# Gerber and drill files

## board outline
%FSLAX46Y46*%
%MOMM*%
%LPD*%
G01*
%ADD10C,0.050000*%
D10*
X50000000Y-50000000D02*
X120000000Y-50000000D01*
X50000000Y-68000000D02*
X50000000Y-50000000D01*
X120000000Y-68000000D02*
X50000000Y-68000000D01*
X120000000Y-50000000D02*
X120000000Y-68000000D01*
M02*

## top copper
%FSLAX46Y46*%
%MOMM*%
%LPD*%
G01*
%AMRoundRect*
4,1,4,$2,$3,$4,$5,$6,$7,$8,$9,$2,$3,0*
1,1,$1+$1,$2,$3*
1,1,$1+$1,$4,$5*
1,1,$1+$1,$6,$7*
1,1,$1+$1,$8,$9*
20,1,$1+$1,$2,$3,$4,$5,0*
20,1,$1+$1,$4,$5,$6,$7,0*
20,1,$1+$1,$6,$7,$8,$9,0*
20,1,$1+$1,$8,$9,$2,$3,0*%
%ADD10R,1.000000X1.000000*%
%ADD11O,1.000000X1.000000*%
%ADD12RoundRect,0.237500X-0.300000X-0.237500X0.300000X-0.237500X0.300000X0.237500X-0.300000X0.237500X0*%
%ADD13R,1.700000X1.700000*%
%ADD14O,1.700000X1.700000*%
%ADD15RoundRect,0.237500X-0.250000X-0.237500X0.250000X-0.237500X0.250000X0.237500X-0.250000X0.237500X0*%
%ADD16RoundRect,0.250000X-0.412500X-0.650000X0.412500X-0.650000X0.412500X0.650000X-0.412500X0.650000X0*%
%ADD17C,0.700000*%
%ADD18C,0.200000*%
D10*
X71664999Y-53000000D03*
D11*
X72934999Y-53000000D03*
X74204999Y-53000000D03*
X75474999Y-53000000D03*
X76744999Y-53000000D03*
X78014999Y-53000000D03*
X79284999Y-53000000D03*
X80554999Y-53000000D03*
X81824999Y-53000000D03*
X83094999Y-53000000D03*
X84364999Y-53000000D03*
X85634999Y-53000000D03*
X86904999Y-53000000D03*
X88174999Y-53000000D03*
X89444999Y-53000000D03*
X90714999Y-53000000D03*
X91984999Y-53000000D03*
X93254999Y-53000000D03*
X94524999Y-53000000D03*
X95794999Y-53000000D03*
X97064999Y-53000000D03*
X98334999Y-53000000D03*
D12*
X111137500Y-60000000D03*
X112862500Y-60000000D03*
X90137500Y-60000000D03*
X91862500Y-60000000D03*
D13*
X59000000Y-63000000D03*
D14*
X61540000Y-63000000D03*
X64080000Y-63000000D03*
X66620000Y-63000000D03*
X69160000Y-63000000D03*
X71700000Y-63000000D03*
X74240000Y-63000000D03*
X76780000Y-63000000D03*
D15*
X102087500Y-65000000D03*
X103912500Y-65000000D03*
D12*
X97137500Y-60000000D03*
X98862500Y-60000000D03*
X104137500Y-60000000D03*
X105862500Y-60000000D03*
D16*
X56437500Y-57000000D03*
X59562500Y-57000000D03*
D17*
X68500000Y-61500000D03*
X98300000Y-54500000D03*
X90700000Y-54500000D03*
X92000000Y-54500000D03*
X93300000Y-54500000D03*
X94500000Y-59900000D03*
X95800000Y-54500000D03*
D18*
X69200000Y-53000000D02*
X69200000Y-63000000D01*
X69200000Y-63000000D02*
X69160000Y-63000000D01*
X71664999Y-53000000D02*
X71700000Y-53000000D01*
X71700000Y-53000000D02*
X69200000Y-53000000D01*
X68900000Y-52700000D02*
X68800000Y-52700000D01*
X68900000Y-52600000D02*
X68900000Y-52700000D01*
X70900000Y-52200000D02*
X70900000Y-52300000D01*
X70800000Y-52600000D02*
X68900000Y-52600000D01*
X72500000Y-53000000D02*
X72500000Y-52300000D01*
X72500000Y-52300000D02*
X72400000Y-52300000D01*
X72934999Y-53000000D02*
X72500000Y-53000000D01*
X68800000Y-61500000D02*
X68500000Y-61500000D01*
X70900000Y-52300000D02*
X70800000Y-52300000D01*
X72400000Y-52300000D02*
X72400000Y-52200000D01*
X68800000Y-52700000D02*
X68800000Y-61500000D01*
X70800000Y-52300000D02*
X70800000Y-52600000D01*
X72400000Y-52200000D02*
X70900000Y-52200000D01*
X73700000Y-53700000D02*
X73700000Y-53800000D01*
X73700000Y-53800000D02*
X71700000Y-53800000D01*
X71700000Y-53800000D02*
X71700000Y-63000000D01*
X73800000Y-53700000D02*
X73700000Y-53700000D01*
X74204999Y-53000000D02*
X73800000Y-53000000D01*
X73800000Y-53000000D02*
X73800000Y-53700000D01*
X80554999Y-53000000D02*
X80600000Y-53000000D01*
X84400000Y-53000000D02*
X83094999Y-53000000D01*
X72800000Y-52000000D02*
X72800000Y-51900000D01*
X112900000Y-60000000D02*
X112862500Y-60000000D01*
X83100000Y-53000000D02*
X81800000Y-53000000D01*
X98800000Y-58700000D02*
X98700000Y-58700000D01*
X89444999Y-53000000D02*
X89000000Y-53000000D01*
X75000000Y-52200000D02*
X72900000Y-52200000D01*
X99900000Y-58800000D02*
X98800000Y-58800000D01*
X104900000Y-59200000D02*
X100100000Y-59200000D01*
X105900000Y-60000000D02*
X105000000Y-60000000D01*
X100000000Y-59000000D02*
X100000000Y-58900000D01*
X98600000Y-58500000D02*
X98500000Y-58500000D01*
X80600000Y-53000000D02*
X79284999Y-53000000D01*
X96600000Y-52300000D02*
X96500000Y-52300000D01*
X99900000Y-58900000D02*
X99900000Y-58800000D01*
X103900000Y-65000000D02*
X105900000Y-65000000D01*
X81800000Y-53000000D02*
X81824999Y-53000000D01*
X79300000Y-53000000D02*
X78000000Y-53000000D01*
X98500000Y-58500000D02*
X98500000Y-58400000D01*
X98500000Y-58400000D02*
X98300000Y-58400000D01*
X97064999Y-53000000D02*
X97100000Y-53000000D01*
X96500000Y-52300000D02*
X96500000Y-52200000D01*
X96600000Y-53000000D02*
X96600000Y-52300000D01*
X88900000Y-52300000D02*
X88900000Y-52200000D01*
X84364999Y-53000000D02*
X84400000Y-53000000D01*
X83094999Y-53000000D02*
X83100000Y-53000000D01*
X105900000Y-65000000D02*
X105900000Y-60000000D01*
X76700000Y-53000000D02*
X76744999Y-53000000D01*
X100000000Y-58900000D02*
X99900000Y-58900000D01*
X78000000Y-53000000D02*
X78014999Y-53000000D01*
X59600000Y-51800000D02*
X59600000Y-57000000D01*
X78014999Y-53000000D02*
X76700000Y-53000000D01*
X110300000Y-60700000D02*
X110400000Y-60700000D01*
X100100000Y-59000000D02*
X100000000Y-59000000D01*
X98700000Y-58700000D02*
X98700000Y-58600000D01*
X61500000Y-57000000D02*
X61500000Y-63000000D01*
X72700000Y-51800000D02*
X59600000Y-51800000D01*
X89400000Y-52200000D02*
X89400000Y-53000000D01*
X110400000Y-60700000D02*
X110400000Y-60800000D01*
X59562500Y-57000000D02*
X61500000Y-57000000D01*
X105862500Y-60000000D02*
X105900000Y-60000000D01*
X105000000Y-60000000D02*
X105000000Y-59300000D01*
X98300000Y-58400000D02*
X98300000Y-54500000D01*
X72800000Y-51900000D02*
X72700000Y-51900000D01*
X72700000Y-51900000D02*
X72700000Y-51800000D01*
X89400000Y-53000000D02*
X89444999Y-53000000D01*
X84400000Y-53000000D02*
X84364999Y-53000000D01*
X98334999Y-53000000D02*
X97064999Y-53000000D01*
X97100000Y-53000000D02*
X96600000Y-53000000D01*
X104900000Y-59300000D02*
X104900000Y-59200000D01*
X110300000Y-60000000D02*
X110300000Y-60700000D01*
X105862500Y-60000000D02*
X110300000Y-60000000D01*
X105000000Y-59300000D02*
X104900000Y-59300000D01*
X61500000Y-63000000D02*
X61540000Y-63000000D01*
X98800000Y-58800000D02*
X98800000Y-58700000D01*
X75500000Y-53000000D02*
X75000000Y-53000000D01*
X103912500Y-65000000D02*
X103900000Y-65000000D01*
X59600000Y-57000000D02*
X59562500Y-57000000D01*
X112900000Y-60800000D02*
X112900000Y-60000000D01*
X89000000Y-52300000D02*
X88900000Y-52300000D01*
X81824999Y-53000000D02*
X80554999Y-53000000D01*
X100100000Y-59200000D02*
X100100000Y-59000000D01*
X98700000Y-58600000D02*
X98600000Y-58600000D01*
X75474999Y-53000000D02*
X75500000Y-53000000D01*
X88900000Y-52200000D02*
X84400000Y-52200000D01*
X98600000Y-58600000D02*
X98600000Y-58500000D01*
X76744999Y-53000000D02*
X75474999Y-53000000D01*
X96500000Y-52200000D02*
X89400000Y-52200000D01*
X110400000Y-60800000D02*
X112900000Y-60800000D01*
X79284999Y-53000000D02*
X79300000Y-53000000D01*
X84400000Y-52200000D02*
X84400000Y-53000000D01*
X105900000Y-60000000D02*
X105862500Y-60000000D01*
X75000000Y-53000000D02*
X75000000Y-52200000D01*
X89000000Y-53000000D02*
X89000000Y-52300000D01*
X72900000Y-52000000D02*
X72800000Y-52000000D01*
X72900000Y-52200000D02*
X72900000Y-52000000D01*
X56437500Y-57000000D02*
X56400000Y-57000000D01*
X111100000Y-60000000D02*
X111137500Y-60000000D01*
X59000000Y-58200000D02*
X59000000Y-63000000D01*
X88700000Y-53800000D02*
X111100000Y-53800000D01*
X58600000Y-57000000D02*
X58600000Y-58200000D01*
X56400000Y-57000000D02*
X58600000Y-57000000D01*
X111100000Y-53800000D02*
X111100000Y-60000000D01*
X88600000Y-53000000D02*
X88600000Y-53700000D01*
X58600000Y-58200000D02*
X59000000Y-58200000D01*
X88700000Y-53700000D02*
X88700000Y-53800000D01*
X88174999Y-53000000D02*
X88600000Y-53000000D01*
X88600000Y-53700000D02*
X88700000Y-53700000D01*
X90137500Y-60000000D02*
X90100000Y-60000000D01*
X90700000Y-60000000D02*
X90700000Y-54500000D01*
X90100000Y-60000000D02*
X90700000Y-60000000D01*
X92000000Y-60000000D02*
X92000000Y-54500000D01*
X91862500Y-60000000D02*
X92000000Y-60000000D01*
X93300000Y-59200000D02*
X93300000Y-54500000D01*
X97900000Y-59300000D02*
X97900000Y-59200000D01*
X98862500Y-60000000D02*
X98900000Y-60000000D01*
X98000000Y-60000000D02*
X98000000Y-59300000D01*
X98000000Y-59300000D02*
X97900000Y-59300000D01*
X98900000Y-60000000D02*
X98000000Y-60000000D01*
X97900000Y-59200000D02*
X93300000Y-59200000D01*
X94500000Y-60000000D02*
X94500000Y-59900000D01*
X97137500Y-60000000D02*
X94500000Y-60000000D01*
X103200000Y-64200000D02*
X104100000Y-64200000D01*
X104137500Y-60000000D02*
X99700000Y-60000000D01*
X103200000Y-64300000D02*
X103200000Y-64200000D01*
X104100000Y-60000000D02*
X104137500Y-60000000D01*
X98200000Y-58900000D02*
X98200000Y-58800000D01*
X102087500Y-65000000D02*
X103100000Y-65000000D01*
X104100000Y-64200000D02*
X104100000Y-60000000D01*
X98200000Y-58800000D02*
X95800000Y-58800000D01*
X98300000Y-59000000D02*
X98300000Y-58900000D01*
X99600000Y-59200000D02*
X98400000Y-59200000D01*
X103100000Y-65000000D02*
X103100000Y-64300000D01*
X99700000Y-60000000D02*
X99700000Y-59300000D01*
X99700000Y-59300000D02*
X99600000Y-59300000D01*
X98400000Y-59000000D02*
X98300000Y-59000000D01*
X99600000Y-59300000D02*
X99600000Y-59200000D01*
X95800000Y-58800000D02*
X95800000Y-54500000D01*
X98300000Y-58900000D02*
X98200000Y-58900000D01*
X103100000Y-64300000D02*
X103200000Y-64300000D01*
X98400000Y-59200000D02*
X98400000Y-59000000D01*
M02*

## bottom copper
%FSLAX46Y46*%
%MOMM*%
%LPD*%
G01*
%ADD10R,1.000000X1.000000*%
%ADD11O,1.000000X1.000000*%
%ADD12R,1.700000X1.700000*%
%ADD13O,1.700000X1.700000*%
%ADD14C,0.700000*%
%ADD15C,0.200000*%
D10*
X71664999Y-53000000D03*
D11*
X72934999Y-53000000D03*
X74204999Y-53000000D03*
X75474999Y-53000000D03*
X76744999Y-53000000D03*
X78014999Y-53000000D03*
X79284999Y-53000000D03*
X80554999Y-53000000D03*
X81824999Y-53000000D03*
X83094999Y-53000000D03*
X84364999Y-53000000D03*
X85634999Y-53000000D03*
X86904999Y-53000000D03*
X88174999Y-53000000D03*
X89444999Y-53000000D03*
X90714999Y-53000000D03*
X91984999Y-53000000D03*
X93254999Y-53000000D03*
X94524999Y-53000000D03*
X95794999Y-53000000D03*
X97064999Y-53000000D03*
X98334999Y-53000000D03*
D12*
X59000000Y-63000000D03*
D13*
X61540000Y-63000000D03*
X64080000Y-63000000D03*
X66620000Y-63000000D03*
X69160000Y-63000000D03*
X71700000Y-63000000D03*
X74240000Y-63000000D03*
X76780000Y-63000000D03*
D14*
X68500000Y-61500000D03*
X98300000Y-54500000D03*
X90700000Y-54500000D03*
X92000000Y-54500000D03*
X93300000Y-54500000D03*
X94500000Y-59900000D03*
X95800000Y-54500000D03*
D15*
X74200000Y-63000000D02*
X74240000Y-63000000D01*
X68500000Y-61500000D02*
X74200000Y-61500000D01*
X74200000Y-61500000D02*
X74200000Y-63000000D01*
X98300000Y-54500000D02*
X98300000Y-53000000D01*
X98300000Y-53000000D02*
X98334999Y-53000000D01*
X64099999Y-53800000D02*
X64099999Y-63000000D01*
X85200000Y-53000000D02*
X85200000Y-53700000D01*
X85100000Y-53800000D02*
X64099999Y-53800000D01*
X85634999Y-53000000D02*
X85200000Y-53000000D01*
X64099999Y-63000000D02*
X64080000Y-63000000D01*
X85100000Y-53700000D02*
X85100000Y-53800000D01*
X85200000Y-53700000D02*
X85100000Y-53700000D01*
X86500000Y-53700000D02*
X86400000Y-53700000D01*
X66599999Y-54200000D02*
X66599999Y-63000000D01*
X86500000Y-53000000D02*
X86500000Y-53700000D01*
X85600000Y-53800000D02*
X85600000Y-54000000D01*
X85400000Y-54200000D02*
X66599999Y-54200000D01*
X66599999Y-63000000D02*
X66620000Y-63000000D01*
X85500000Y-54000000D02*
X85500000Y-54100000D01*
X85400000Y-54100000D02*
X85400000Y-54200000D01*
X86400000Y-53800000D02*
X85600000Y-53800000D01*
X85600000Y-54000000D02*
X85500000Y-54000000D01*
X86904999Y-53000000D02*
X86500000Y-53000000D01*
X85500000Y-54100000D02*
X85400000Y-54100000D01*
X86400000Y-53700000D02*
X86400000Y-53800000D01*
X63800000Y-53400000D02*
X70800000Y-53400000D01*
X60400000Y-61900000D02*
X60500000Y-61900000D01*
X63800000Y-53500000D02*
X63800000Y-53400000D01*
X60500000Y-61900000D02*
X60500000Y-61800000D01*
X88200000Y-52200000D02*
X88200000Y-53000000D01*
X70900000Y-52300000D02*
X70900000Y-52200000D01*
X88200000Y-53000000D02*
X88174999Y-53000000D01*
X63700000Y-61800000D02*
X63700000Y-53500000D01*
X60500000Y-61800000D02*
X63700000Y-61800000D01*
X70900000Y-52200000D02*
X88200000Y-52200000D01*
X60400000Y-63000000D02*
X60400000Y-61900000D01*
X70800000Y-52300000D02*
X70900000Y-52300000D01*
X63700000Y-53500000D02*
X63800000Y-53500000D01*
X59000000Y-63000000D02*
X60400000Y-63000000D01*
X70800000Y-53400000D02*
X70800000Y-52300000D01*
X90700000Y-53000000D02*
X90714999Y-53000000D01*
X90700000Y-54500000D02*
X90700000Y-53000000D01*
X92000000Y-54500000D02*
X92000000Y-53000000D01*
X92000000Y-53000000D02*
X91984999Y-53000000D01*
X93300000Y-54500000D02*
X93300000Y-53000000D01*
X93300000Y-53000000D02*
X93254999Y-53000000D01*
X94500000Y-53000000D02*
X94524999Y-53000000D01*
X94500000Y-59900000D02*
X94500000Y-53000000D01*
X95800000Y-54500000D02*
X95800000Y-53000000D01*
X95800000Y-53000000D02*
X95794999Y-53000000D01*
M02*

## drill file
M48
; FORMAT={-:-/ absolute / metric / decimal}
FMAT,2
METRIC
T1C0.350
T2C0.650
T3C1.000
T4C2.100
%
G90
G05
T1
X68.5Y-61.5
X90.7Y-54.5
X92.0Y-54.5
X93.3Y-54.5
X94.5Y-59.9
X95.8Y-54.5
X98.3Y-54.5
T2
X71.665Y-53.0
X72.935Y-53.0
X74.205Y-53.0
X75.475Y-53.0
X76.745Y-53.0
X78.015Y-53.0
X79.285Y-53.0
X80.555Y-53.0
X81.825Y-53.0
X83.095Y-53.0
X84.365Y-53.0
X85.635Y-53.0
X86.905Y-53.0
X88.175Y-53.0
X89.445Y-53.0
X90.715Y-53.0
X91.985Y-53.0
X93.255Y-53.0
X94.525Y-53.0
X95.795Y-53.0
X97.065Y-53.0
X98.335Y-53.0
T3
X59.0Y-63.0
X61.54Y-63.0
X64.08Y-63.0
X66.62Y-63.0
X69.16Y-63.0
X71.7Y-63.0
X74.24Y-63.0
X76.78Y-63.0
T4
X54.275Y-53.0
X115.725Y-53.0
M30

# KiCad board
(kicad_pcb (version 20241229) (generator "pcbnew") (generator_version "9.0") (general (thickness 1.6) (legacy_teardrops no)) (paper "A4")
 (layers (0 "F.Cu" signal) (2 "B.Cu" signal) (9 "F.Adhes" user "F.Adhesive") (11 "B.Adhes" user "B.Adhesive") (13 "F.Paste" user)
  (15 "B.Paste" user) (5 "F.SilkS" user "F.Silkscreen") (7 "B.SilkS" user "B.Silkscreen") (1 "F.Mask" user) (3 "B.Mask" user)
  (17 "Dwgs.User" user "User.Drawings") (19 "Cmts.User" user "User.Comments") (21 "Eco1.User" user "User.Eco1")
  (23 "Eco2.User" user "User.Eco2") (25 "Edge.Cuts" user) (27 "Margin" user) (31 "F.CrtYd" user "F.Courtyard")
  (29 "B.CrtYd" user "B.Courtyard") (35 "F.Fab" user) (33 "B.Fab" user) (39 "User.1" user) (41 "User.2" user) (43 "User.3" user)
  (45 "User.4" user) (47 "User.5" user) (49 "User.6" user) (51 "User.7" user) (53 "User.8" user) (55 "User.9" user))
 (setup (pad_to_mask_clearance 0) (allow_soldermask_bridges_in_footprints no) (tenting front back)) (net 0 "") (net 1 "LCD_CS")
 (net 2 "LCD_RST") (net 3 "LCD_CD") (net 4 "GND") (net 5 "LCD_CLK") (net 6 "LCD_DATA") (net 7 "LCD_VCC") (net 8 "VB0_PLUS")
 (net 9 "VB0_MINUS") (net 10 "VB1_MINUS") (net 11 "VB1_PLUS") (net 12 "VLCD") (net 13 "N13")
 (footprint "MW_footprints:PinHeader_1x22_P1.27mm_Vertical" (layer "F.Cu") (at 71.664999 53 90)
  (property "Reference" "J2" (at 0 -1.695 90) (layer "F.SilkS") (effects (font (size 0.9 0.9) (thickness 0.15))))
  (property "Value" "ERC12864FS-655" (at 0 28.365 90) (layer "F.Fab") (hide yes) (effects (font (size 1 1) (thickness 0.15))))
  (pad "1" thru_hole rect (at 0 0 90) (size 1 1) (drill 0.65) (layers "*.Cu" "*.Mask") (remove_unused_layers no) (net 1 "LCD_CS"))
  (pad "2" thru_hole oval (at 0 1.27 90) (size 1 1) (drill 0.65) (layers "*.Cu" "*.Mask") (remove_unused_layers no) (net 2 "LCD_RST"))
  (pad "3" thru_hole oval (at 0 2.54 90) (size 1 1) (drill 0.65) (layers "*.Cu" "*.Mask") (remove_unused_layers no) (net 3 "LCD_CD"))
  (pad "4" thru_hole oval (at 0 3.81 90) (size 1 1) (drill 0.65) (layers "*.Cu" "*.Mask") (remove_unused_layers no) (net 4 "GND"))
  (pad "5" thru_hole oval (at 0 5.08 90) (size 1 1) (drill 0.65) (layers "*.Cu" "*.Mask") (remove_unused_layers no) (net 4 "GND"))
  (pad "6" thru_hole oval (at 0 6.35 90) (size 1 1) (drill 0.65) (layers "*.Cu" "*.Mask") (remove_unused_layers no) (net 4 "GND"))
  (pad "7" thru_hole oval (at 0 7.62 90) (size 1 1) (drill 0.65) (layers "*.Cu" "*.Mask") (remove_unused_layers no) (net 4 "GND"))
  (pad "8" thru_hole oval (at 0 8.89 90) (size 1 1) (drill 0.65) (layers "*.Cu" "*.Mask") (remove_unused_layers no) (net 4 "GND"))
  (pad "9" thru_hole oval (at 0 10.16 90) (size 1 1) (drill 0.65) (layers "*.Cu" "*.Mask") (remove_unused_layers no) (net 4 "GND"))
  (pad "10" thru_hole oval (at 0 11.43 90) (size 1 1) (drill 0.65) (layers "*.Cu" "*.Mask") (remove_unused_layers no) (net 4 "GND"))
  (pad "11" thru_hole oval (at 0 12.7 90) (size 1 1) (drill 0.65) (layers "*.Cu" "*.Mask") (remove_unused_layers no) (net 4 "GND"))
  (pad "12" thru_hole oval (at 0 13.97 90) (size 1 1) (drill 0.65) (layers "*.Cu" "*.Mask") (remove_unused_layers no) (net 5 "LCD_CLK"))
  (pad "13" thru_hole oval (at 0 15.24 90) (size 1 1) (drill 0.65) (layers "*.Cu" "*.Mask") (remove_unused_layers no) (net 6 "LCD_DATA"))
  (pad "14" thru_hole oval (at 0 16.51 90) (size 1 1) (drill 0.65) (layers "*.Cu" "*.Mask") (remove_unused_layers no) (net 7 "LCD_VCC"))
  (pad "15" thru_hole oval (at 0 17.78 90) (size 1 1) (drill 0.65) (layers "*.Cu" "*.Mask") (remove_unused_layers no) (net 4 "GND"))
  (pad "16" thru_hole oval (at 0 19.05 90) (size 1 1) (drill 0.65) (layers "*.Cu" "*.Mask") (remove_unused_layers no) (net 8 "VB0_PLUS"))
  (pad "17" thru_hole oval (at 0 20.32 90) (size 1 1) (drill 0.65) (layers "*.Cu" "*.Mask") (remove_unused_layers no) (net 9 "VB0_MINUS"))
  (pad "18" thru_hole oval (at 0 21.59 90) (size 1 1) (drill 0.65) (layers "*.Cu" "*.Mask") (remove_unused_layers no) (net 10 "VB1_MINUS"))
  (pad "19" thru_hole oval (at 0 22.86 90) (size 1 1) (drill 0.65) (layers "*.Cu" "*.Mask") (remove_unused_layers no) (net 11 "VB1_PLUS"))
  (pad "20" thru_hole oval (at 0 24.13 90) (size 1 1) (drill 0.65) (layers "*.Cu" "*.Mask") (remove_unused_layers no) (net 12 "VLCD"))
  (pad "21" thru_hole oval (at 0 25.4 90) (size 1 1) (drill 0.65) (layers "*.Cu" "*.Mask") (remove_unused_layers no) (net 4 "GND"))
  (pad "22" thru_hole oval (at 0 26.67 90) (size 1 1) (drill 0.65) (layers "*.Cu" "*.Mask") (remove_unused_layers no) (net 4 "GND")))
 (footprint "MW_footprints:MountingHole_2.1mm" (layer "F.Cu") (at 54.275 53)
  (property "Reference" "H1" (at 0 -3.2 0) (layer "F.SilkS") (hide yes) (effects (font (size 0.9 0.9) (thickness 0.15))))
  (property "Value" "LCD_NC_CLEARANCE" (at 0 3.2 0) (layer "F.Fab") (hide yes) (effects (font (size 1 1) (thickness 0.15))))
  (pad "" np_thru_hole circle (at 0 0) (size 2.1 2.1) (drill 2.1) (layers "*.Cu" "*.Mask")))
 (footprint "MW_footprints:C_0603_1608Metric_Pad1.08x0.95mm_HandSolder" (layer "F.Cu") (at 112 60)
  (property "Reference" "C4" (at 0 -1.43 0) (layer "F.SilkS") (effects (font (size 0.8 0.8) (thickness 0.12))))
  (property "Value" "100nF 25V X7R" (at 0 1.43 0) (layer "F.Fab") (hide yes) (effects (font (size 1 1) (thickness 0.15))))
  (pad "1" smd roundrect (at -0.8625 0) (size 1.075 0.95) (layers "F.Cu" "F.Mask" "F.Paste") (roundrect_rratio 0.25) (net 7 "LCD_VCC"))
  (pad "2" smd roundrect (at 0.8625 0) (size 1.075 0.95) (layers "F.Cu" "F.Mask" "F.Paste") (roundrect_rratio 0.25) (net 4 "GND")))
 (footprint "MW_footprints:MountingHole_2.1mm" (layer "F.Cu") (at 115.725 53)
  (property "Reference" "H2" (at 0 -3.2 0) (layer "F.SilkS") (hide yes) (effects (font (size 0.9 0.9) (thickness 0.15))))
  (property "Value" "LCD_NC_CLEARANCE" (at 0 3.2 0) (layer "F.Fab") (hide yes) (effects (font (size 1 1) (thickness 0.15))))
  (pad "" np_thru_hole circle (at 0 0) (size 2.1 2.1) (drill 2.1) (layers "*.Cu" "*.Mask")))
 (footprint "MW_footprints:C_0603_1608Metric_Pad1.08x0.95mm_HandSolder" (layer "F.Cu") (at 91 60)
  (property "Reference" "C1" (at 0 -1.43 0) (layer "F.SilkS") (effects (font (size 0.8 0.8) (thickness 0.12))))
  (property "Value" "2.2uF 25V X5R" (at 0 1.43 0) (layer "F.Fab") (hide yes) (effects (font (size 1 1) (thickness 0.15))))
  (pad "1" smd roundrect (at -0.8625 0) (size 1.075 0.95) (layers "F.Cu" "F.Mask" "F.Paste") (roundrect_rratio 0.25) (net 8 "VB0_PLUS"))
  (pad "2" smd roundrect (at 0.8625 0) (size 1.075 0.95) (layers "F.Cu" "F.Mask" "F.Paste") (roundrect_rratio 0.25) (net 9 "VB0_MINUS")))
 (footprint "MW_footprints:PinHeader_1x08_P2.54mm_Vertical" (layer "F.Cu") (at 59 63 90)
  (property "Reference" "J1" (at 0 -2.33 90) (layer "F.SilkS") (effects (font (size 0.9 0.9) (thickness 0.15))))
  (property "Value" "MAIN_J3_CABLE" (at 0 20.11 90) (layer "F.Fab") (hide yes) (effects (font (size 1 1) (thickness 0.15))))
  (pad "1" thru_hole rect (at 0 0 90) (size 1.7 1.7) (drill 1) (layers "*.Cu" "*.Mask") (remove_unused_layers no) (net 7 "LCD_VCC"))
  (pad "2" thru_hole oval (at 0 2.54 90) (size 1.7 1.7) (drill 1) (layers "*.Cu" "*.Mask") (remove_unused_layers no) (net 4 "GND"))
  (pad "3" thru_hole oval (at 0 5.08 90) (size 1.7 1.7) (drill 1) (layers "*.Cu" "*.Mask") (remove_unused_layers no) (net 5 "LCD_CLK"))
  (pad "4" thru_hole oval (at 0 7.62 90) (size 1.7 1.7) (drill 1) (layers "*.Cu" "*.Mask") (remove_unused_layers no) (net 6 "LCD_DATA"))
  (pad "5" thru_hole oval (at 0 10.16 90) (size 1.7 1.7) (drill 1) (layers "*.Cu" "*.Mask") (remove_unused_layers no) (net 1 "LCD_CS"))
  (pad "6" thru_hole oval (at 0 12.7 90) (size 1.7 1.7) (drill 1) (layers "*.Cu" "*.Mask") (remove_unused_layers no) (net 3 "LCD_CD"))
  (pad "7" thru_hole oval (at 0 15.24 90) (size 1.7 1.7) (drill 1) (layers "*.Cu" "*.Mask") (remove_unused_layers no) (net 2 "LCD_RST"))
  (pad "8" thru_hole oval (at 0 17.78 90) (size 1.7 1.7) (drill 1) (layers "*.Cu" "*.Mask") (remove_unused_layers no) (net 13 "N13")))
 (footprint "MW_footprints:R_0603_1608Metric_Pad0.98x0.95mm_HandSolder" (layer "F.Cu") (at 103 65)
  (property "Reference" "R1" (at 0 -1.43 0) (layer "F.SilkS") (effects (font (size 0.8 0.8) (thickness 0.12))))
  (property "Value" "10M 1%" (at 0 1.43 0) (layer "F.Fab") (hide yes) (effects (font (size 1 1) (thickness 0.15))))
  (pad "1" smd roundrect (at -0.9125 0) (size 0.975 0.95) (layers "F.Cu" "F.Mask" "F.Paste") (roundrect_rratio 0.25) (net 12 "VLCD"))
  (pad "2" smd roundrect (at 0.9125 0) (size 0.975 0.95) (layers "F.Cu" "F.Mask" "F.Paste") (roundrect_rratio 0.25) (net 4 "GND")))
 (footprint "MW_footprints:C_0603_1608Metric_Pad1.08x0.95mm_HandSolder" (layer "F.Cu") (at 98 60)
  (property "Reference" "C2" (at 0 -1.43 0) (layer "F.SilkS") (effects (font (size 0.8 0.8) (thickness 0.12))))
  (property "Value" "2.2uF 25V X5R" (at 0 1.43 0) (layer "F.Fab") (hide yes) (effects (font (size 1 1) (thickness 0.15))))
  (pad "1" smd roundrect (at -0.8625 0) (size 1.075 0.95) (layers "F.Cu" "F.Mask" "F.Paste") (roundrect_rratio 0.25) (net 11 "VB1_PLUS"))
  (pad "2" smd roundrect (at 0.8625 0) (size 1.075 0.95) (layers "F.Cu" "F.Mask" "F.Paste") (roundrect_rratio 0.25) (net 10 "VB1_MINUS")))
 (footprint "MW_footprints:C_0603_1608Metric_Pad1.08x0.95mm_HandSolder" (layer "F.Cu") (at 105 60)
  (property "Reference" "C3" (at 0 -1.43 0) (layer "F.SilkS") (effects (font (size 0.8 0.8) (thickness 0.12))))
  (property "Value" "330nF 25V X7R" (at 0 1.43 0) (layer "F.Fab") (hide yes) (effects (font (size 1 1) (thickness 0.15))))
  (pad "1" smd roundrect (at -0.8625 0) (size 1.075 0.95) (layers "F.Cu" "F.Mask" "F.Paste") (roundrect_rratio 0.25) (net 12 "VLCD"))
  (pad "2" smd roundrect (at 0.8625 0) (size 1.075 0.95) (layers "F.Cu" "F.Mask" "F.Paste") (roundrect_rratio 0.25) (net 4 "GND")))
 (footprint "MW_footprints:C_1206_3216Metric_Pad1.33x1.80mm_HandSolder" (layer "F.Cu") (at 58 57)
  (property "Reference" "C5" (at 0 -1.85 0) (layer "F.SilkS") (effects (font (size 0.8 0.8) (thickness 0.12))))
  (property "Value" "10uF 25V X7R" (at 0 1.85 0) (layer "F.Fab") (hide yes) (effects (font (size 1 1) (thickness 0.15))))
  (pad "1" smd roundrect (at -1.5625 0) (size 1.325 1.8) (layers "F.Cu" "F.Mask" "F.Paste") (roundrect_rratio 0.188679) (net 7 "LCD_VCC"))
  (pad "2" smd roundrect (at 1.5625 0) (size 1.325 1.8) (layers "F.Cu" "F.Mask" "F.Paste") (roundrect_rratio 0.188679) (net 4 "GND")))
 (gr_line (start 50 50) (end 120 50) (stroke (width 0.05) (type default)) (layer "Edge.Cuts"))
 (gr_line (start 50 68) (end 50 50) (stroke (width 0.05) (type default)) (layer "Edge.Cuts"))
 (gr_line (start 120 68) (end 50 68) (stroke (width 0.05) (type default)) (layer "Edge.Cuts"))
 (gr_line (start 120 50) (end 120 68) (stroke (width 0.05) (type default)) (layer "Edge.Cuts"))
 (segment (start 69.2 53) (end 69.2 63) (width 0.2) (layer "F.Cu") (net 1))
 (segment (start 69.2 63) (end 69.16 63) (width 0.2) (layer "F.Cu") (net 1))
 (segment (start 71.664999 53) (end 71.7 53) (width 0.2) (layer "F.Cu") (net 1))
 (segment (start 71.7 53) (end 69.2 53) (width 0.2) (layer "F.Cu") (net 1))
 (segment (start 68.9 52.7) (end 68.8 52.7) (width 0.2) (layer "F.Cu") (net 2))
 (segment (start 68.9 52.6) (end 68.9 52.7) (width 0.2) (layer "F.Cu") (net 2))
 (segment (start 70.9 52.2) (end 70.9 52.3) (width 0.2) (layer "F.Cu") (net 2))
 (segment (start 70.8 52.6) (end 68.9 52.6) (width 0.2) (layer "F.Cu") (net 2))
 (segment (start 72.5 53) (end 72.5 52.3) (width 0.2) (layer "F.Cu") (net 2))
 (segment (start 72.5 52.3) (end 72.4 52.3) (width 0.2) (layer "F.Cu") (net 2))
 (segment (start 72.934999 53) (end 72.5 53) (width 0.2) (layer "F.Cu") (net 2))
 (segment (start 68.8 61.5) (end 68.5 61.5) (width 0.2) (layer "F.Cu") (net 2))
 (segment (start 70.9 52.3) (end 70.8 52.3) (width 0.2) (layer "F.Cu") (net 2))
 (segment (start 72.4 52.3) (end 72.4 52.2) (width 0.2) (layer "F.Cu") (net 2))
 (segment (start 68.8 52.7) (end 68.8 61.5) (width 0.2) (layer "F.Cu") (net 2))
 (segment (start 70.8 52.3) (end 70.8 52.6) (width 0.2) (layer "F.Cu") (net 2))
 (segment (start 72.4 52.2) (end 70.9 52.2) (width 0.2) (layer "F.Cu") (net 2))
 (via (at 68.5 61.5) (size 0.7) (drill 0.35) (layers "F.Cu" "B.Cu") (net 2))
 (segment (start 74.2 63) (end 74.24 63) (width 0.2) (layer "B.Cu") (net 2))
 (segment (start 68.5 61.5) (end 74.2 61.5) (width 0.2) (layer "B.Cu") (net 2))
 (segment (start 74.2 61.5) (end 74.2 63) (width 0.2) (layer "B.Cu") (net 2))
 (segment (start 73.7 53.7) (end 73.7 53.8) (width 0.2) (layer "F.Cu") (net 3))
 (segment (start 73.7 53.8) (end 71.7 53.8) (width 0.2) (layer "F.Cu") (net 3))
 (segment (start 71.7 53.8) (end 71.7 63) (width 0.2) (layer "F.Cu") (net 3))
 (segment (start 73.8 53.7) (end 73.7 53.7) (width 0.2) (layer "F.Cu") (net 3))
 (segment (start 74.204999 53) (end 73.8 53) (width 0.2) (layer "F.Cu") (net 3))
 (segment (start 73.8 53) (end 73.8 53.7) (width 0.2) (layer "F.Cu") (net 3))
 (segment (start 80.554999 53) (end 80.6 53) (width 0.2) (layer "F.Cu") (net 4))
 (segment (start 84.4 53) (end 83.094999 53) (width 0.2) (layer "F.Cu") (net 4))
 (segment (start 72.8 52) (end 72.8 51.9) (width 0.2) (layer "F.Cu") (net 4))
 (segment (start 112.9 60) (end 112.8625 60) (width 0.2) (layer "F.Cu") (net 4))
 (segment (start 83.1 53) (end 81.8 53) (width 0.2) (layer "F.Cu") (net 4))
 (segment (start 98.8 58.7) (end 98.7 58.7) (width 0.2) (layer "F.Cu") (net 4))
 (segment (start 89.444999 53) (end 89 53) (width 0.2) (layer "F.Cu") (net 4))
 (segment (start 75 52.2) (end 72.9 52.2) (width 0.2) (layer "F.Cu") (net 4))
 (segment (start 99.9 58.8) (end 98.8 58.8) (width 0.2) (layer "F.Cu") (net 4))
 (segment (start 104.9 59.2) (end 100.1 59.2) (width 0.2) (layer "F.Cu") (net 4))
 (segment (start 105.9 60) (end 105 60) (width 0.2) (layer "F.Cu") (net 4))
 (segment (start 100 59) (end 100 58.9) (width 0.2) (layer "F.Cu") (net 4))
 (segment (start 98.6 58.5) (end 98.5 58.5) (width 0.2) (layer "F.Cu") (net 4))
 (segment (start 80.6 53) (end 79.284999 53) (width 0.2) (layer "F.Cu") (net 4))
 (segment (start 96.6 52.3) (end 96.5 52.3) (width 0.2) (layer "F.Cu") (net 4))
 (segment (start 99.9 58.9) (end 99.9 58.8) (width 0.2) (layer "F.Cu") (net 4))
 (segment (start 103.9 65) (end 105.9 65) (width 0.2) (layer "F.Cu") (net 4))
 (segment (start 81.8 53) (end 81.824999 53) (width 0.2) (layer "F.Cu") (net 4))
 (segment (start 79.3 53) (end 78 53) (width 0.2) (layer "F.Cu") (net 4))
 (segment (start 98.5 58.5) (end 98.5 58.4) (width 0.2) (layer "F.Cu") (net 4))
 (segment (start 98.5 58.4) (end 98.3 58.4) (width 0.2) (layer "F.Cu") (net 4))
 (segment (start 97.064999 53) (end 97.1 53) (width 0.2) (layer "F.Cu") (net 4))
 (segment (start 96.5 52.3) (end 96.5 52.2) (width 0.2) (layer "F.Cu") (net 4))
 (segment (start 96.6 53) (end 96.6 52.3) (width 0.2) (layer "F.Cu") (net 4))
 (segment (start 88.9 52.3) (end 88.9 52.2) (width 0.2) (layer "F.Cu") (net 4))
 (segment (start 84.364999 53) (end 84.4 53) (width 0.2) (layer "F.Cu") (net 4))
 (segment (start 83.094999 53) (end 83.1 53) (width 0.2) (layer "F.Cu") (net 4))
 (segment (start 105.9 65) (end 105.9 60) (width 0.2) (layer "F.Cu") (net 4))
 (segment (start 76.7 53) (end 76.744999 53) (width 0.2) (layer "F.Cu") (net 4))
 (segment (start 100 58.9) (end 99.9 58.9) (width 0.2) (layer "F.Cu") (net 4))
 (segment (start 78 53) (end 78.014999 53) (width 0.2) (layer "F.Cu") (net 4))
 (segment (start 59.6 51.8) (end 59.6 57) (width 0.2) (layer "F.Cu") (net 4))
 (segment (start 78.014999 53) (end 76.7 53) (width 0.2) (layer "F.Cu") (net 4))
 (segment (start 110.3 60.7) (end 110.4 60.7) (width 0.2) (layer "F.Cu") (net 4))
 (segment (start 100.1 59) (end 100 59) (width 0.2) (layer "F.Cu") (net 4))
 (segment (start 98.7 58.7) (end 98.7 58.6) (width 0.2) (layer "F.Cu") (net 4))
 (segment (start 61.5 57) (end 61.5 63) (width 0.2) (layer "F.Cu") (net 4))
 (segment (start 72.7 51.8) (end 59.6 51.8) (width 0.2) (layer "F.Cu") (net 4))
 (segment (start 89.4 52.2) (end 89.4 53) (width 0.2) (layer "F.Cu") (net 4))
 (segment (start 110.4 60.7) (end 110.4 60.8) (width 0.2) (layer "F.Cu") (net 4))
 (segment (start 59.5625 57) (end 61.5 57) (width 0.2) (layer "F.Cu") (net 4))
 (segment (start 105.8625 60) (end 105.9 60) (width 0.2) (layer "F.Cu") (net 4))
 (segment (start 105 60) (end 105 59.3) (width 0.2) (layer "F.Cu") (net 4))
 (segment (start 98.3 58.4) (end 98.3 54.5) (width 0.2) (layer "F.Cu") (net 4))
 (segment (start 72.8 51.9) (end 72.7 51.9) (width 0.2) (layer "F.Cu") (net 4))
 (segment (start 72.7 51.9) (end 72.7 51.8) (width 0.2) (layer "F.Cu") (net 4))
 (segment (start 89.4 53) (end 89.444999 53) (width 0.2) (layer "F.Cu") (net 4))
 (segment (start 84.4 53) (end 84.364999 53) (width 0.2) (layer "F.Cu") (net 4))
 (segment (start 98.334999 53) (end 97.064999 53) (width 0.2) (layer "F.Cu") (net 4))
 (segment (start 97.1 53) (end 96.6 53) (width 0.2) (layer "F.Cu") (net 4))
 (segment (start 104.9 59.3) (end 104.9 59.2) (width 0.2) (layer "F.Cu") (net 4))
 (segment (start 110.3 60) (end 110.3 60.7) (width 0.2) (layer "F.Cu") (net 4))
 (segment (start 105.8625 60) (end 110.3 60) (width 0.2) (layer "F.Cu") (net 4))
 (segment (start 105 59.3) (end 104.9 59.3) (width 0.2) (layer "F.Cu") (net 4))
 (segment (start 61.5 63) (end 61.54 63) (width 0.2) (layer "F.Cu") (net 4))
 (segment (start 98.8 58.8) (end 98.8 58.7) (width 0.2) (layer "F.Cu") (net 4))
 (segment (start 75.5 53) (end 75 53) (width 0.2) (layer "F.Cu") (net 4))
 (segment (start 103.9125 65) (end 103.9 65) (width 0.2) (layer "F.Cu") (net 4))
 (segment (start 59.6 57) (end 59.5625 57) (width 0.2) (layer "F.Cu") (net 4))
 (segment (start 112.9 60.8) (end 112.9 60) (width 0.2) (layer "F.Cu") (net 4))
 (segment (start 89 52.3) (end 88.9 52.3) (width 0.2) (layer "F.Cu") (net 4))
 (segment (start 81.824999 53) (end 80.554999 53) (width 0.2) (layer "F.Cu") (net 4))
 (segment (start 100.1 59.2) (end 100.1 59) (width 0.2) (layer "F.Cu") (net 4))
 (segment (start 98.7 58.6) (end 98.6 58.6) (width 0.2) (layer "F.Cu") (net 4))
 (segment (start 75.474999 53) (end 75.5 53) (width 0.2) (layer "F.Cu") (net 4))
 (segment (start 88.9 52.2) (end 84.4 52.2) (width 0.2) (layer "F.Cu") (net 4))
 (segment (start 98.6 58.6) (end 98.6 58.5) (width 0.2) (layer "F.Cu") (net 4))
 (segment (start 76.744999 53) (end 75.474999 53) (width 0.2) (layer "F.Cu") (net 4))
 (segment (start 96.5 52.2) (end 89.4 52.2) (width 0.2) (layer "F.Cu") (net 4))
 (segment (start 110.4 60.8) (end 112.9 60.8) (width 0.2) (layer "F.Cu") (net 4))
 (segment (start 79.284999 53) (end 79.3 53) (width 0.2) (layer "F.Cu") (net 4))
 (segment (start 84.4 52.2) (end 84.4 53) (width 0.2) (layer "F.Cu") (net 4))
 (segment (start 105.9 60) (end 105.8625 60) (width 0.2) (layer "F.Cu") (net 4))
 (segment (start 75 53) (end 75 52.2) (width 0.2) (layer "F.Cu") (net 4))
 (segment (start 89 53) (end 89 52.3) (width 0.2) (layer "F.Cu") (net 4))
 (segment (start 72.9 52) (end 72.8 52) (width 0.2) (layer "F.Cu") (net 4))
 (segment (start 72.9 52.2) (end 72.9 52) (width 0.2) (layer "F.Cu") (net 4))
 (via (at 98.3 54.5) (size 0.7) (drill 0.35) (layers "F.Cu" "B.Cu") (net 4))
 (segment (start 98.3 54.5) (end 98.3 53) (width 0.2) (layer "B.Cu") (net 4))
 (segment (start 98.3 53) (end 98.334999 53) (width 0.2) (layer "B.Cu") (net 4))
 (segment (start 64.099999 53.8) (end 64.099999 63) (width 0.2) (layer "B.Cu") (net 5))
 (segment (start 85.2 53) (end 85.2 53.7) (width 0.2) (layer "B.Cu") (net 5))
 (segment (start 85.1 53.8) (end 64.099999 53.8) (width 0.2) (layer "B.Cu") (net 5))
 (segment (start 85.634999 53) (end 85.2 53) (width 0.2) (layer "B.Cu") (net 5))
 (segment (start 64.099999 63) (end 64.08 63) (width 0.2) (layer "B.Cu") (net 5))
 (segment (start 85.1 53.7) (end 85.1 53.8) (width 0.2) (layer "B.Cu") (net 5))
 (segment (start 85.2 53.7) (end 85.1 53.7) (width 0.2) (layer "B.Cu") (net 5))
 (segment (start 86.5 53.7) (end 86.4 53.7) (width 0.2) (layer "B.Cu") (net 6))
 (segment (start 66.599999 54.2) (end 66.599999 63) (width 0.2) (layer "B.Cu") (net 6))
 (segment (start 86.5 53) (end 86.5 53.7) (width 0.2) (layer "B.Cu") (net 6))
 (segment (start 85.6 53.8) (end 85.6 54) (width 0.2) (layer "B.Cu") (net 6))
 (segment (start 85.4 54.2) (end 66.599999 54.2) (width 0.2) (layer "B.Cu") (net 6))
 (segment (start 66.599999 63) (end 66.62 63) (width 0.2) (layer "B.Cu") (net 6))
 (segment (start 85.5 54) (end 85.5 54.1) (width 0.2) (layer "B.Cu") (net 6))
 (segment (start 85.4 54.1) (end 85.4 54.2) (width 0.2) (layer "B.Cu") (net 6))
 (segment (start 86.4 53.8) (end 85.6 53.8) (width 0.2) (layer "B.Cu") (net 6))
 (segment (start 85.6 54) (end 85.5 54) (width 0.2) (layer "B.Cu") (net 6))
 (segment (start 86.904999 53) (end 86.5 53) (width 0.2) (layer "B.Cu") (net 6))
 (segment (start 85.5 54.1) (end 85.4 54.1) (width 0.2) (layer "B.Cu") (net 6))
 (segment (start 86.4 53.7) (end 86.4 53.8) (width 0.2) (layer "B.Cu") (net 6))
 (segment (start 56.4375 57) (end 56.4 57) (width 0.2) (layer "F.Cu") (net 7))
 (segment (start 111.1 60) (end 111.1375 60) (width 0.2) (layer "F.Cu") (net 7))
 (segment (start 59 58.2) (end 59 63) (width 0.2) (layer "F.Cu") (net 7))
 (segment (start 88.7 53.8) (end 111.1 53.8) (width 0.2) (layer "F.Cu") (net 7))
 (segment (start 58.6 57) (end 58.6 58.2) (width 0.2) (layer "F.Cu") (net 7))
 (segment (start 56.4 57) (end 58.6 57) (width 0.2) (layer "F.Cu") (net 7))
 (segment (start 111.1 53.8) (end 111.1 60) (width 0.2) (layer "F.Cu") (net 7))
 (segment (start 88.6 53) (end 88.6 53.7) (width 0.2) (layer "F.Cu") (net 7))
 (segment (start 58.6 58.2) (end 59 58.2) (width 0.2) (layer "F.Cu") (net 7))
 (segment (start 88.7 53.7) (end 88.7 53.8) (width 0.2) (layer "F.Cu") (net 7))
 (segment (start 88.174999 53) (end 88.6 53) (width 0.2) (layer "F.Cu") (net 7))
 (segment (start 88.6 53.7) (end 88.7 53.7) (width 0.2) (layer "F.Cu") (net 7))
 (segment (start 63.8 53.4) (end 70.8 53.4) (width 0.2) (layer "B.Cu") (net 7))
 (segment (start 60.4 61.9) (end 60.5 61.9) (width 0.2) (layer "B.Cu") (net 7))
 (segment (start 63.8 53.5) (end 63.8 53.4) (width 0.2) (layer "B.Cu") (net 7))
 (segment (start 60.5 61.9) (end 60.5 61.8) (width 0.2) (layer "B.Cu") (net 7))
 (segment (start 88.2 52.2) (end 88.2 53) (width 0.2) (layer "B.Cu") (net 7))
 (segment (start 70.9 52.3) (end 70.9 52.2) (width 0.2) (layer "B.Cu") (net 7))
 (segment (start 88.2 53) (end 88.174999 53) (width 0.2) (layer "B.Cu") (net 7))
 (segment (start 63.7 61.8) (end 63.7 53.5) (width 0.2) (layer "B.Cu") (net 7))
 (segment (start 60.5 61.8) (end 63.7 61.8) (width 0.2) (layer "B.Cu") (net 7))
 (segment (start 70.9 52.2) (end 88.2 52.2) (width 0.2) (layer "B.Cu") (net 7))
 (segment (start 60.4 63) (end 60.4 61.9) (width 0.2) (layer "B.Cu") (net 7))
 (segment (start 70.8 52.3) (end 70.9 52.3) (width 0.2) (layer "B.Cu") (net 7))
 (segment (start 63.7 53.5) (end 63.8 53.5) (width 0.2) (layer "B.Cu") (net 7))
 (segment (start 59 63) (end 60.4 63) (width 0.2) (layer "B.Cu") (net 7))
 (segment (start 70.8 53.4) (end 70.8 52.3) (width 0.2) (layer "B.Cu") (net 7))
 (segment (start 90.1375 60) (end 90.1 60) (width 0.2) (layer "F.Cu") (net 8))
 (segment (start 90.7 60) (end 90.7 54.5) (width 0.2) (layer "F.Cu") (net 8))
 (segment (start 90.1 60) (end 90.7 60) (width 0.2) (layer "F.Cu") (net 8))
 (via (at 90.7 54.5) (size 0.7) (drill 0.35) (layers "F.Cu" "B.Cu") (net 8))
 (segment (start 90.7 53) (end 90.714999 53) (width 0.2) (layer "B.Cu") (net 8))
 (segment (start 90.7 54.5) (end 90.7 53) (width 0.2) (layer "B.Cu") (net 8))
 (segment (start 92 60) (end 92 54.5) (width 0.2) (layer "F.Cu") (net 9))
 (segment (start 91.8625 60) (end 92 60) (width 0.2) (layer "F.Cu") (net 9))
 (via (at 92 54.5) (size 0.7) (drill 0.35) (layers "F.Cu" "B.Cu") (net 9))
 (segment (start 92 54.5) (end 92 53) (width 0.2) (layer "B.Cu") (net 9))
 (segment (start 92 53) (end 91.984999 53) (width 0.2) (layer "B.Cu") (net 9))
 (segment (start 93.3 59.2) (end 93.3 54.5) (width 0.2) (layer "F.Cu") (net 10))
 (segment (start 97.9 59.3) (end 97.9 59.2) (width 0.2) (layer "F.Cu") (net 10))
 (segment (start 98.8625 60) (end 98.9 60) (width 0.2) (layer "F.Cu") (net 10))
 (segment (start 98 60) (end 98 59.3) (width 0.2) (layer "F.Cu") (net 10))
 (segment (start 98 59.3) (end 97.9 59.3) (width 0.2) (layer "F.Cu") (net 10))
 (segment (start 98.9 60) (end 98 60) (width 0.2) (layer "F.Cu") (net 10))
 (segment (start 97.9 59.2) (end 93.3 59.2) (width 0.2) (layer "F.Cu") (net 10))
 (via (at 93.3 54.5) (size 0.7) (drill 0.35) (layers "F.Cu" "B.Cu") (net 10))
 (segment (start 93.3 54.5) (end 93.3 53) (width 0.2) (layer "B.Cu") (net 10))
 (segment (start 93.3 53) (end 93.254999 53) (width 0.2) (layer "B.Cu") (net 10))
 (segment (start 94.5 60) (end 94.5 59.9) (width 0.2) (layer "F.Cu") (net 11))
 (segment (start 97.1375 60) (end 94.5 60) (width 0.2) (layer "F.Cu") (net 11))
 (via (at 94.5 59.9) (size 0.7) (drill 0.35) (layers "F.Cu" "B.Cu") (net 11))
 (segment (start 94.5 53) (end 94.524999 53) (width 0.2) (layer "B.Cu") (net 11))
 (segment (start 94.5 59.9) (end 94.5 53) (width 0.2) (layer "B.Cu") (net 11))
 (segment (start 103.2 64.2) (end 104.1 64.2) (width 0.2) (layer "F.Cu") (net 12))
 (segment (start 104.1375 60) (end 99.7 60) (width 0.2) (layer "F.Cu") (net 12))
 (segment (start 103.2 64.3) (end 103.2 64.2) (width 0.2) (layer "F.Cu") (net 12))
 (segment (start 104.1 60) (end 104.1375 60) (width 0.2) (layer "F.Cu") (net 12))
 (segment (start 98.2 58.9) (end 98.2 58.8) (width 0.2) (layer "F.Cu") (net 12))
 (segment (start 102.0875 65) (end 103.1 65) (width 0.2) (layer "F.Cu") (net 12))
 (segment (start 104.1 64.2) (end 104.1 60) (width 0.2) (layer "F.Cu") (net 12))
 (segment (start 98.2 58.8) (end 95.8 58.8) (width 0.2) (layer "F.Cu") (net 12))
 (segment (start 98.3 59) (end 98.3 58.9) (width 0.2) (layer "F.Cu") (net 12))
 (segment (start 99.6 59.2) (end 98.4 59.2) (width 0.2) (layer "F.Cu") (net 12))
 (segment (start 103.1 65) (end 103.1 64.3) (width 0.2) (layer "F.Cu") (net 12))
 (segment (start 99.7 60) (end 99.7 59.3) (width 0.2) (layer "F.Cu") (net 12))
 (segment (start 99.7 59.3) (end 99.6 59.3) (width 0.2) (layer "F.Cu") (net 12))
 (segment (start 98.4 59) (end 98.3 59) (width 0.2) (layer "F.Cu") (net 12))
 (segment (start 99.6 59.3) (end 99.6 59.2) (width 0.2) (layer "F.Cu") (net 12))
 (segment (start 95.8 58.8) (end 95.8 54.5) (width 0.2) (layer "F.Cu") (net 12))
 (segment (start 98.3 58.9) (end 98.2 58.9) (width 0.2) (layer "F.Cu") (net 12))
 (segment (start 103.1 64.3) (end 103.2 64.3) (width 0.2) (layer "F.Cu") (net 12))
 (segment (start 98.4 59.2) (end 98.4 59) (width 0.2) (layer "F.Cu") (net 12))
 (via (at 95.8 54.5) (size 0.7) (drill 0.35) (layers "F.Cu" "B.Cu") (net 12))
 (segment (start 95.8 54.5) (end 95.8 53) (width 0.2) (layer "B.Cu") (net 12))
 (segment (start 95.8 53) (end 95.794999 53) (width 0.2) (layer "B.Cu") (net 12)))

